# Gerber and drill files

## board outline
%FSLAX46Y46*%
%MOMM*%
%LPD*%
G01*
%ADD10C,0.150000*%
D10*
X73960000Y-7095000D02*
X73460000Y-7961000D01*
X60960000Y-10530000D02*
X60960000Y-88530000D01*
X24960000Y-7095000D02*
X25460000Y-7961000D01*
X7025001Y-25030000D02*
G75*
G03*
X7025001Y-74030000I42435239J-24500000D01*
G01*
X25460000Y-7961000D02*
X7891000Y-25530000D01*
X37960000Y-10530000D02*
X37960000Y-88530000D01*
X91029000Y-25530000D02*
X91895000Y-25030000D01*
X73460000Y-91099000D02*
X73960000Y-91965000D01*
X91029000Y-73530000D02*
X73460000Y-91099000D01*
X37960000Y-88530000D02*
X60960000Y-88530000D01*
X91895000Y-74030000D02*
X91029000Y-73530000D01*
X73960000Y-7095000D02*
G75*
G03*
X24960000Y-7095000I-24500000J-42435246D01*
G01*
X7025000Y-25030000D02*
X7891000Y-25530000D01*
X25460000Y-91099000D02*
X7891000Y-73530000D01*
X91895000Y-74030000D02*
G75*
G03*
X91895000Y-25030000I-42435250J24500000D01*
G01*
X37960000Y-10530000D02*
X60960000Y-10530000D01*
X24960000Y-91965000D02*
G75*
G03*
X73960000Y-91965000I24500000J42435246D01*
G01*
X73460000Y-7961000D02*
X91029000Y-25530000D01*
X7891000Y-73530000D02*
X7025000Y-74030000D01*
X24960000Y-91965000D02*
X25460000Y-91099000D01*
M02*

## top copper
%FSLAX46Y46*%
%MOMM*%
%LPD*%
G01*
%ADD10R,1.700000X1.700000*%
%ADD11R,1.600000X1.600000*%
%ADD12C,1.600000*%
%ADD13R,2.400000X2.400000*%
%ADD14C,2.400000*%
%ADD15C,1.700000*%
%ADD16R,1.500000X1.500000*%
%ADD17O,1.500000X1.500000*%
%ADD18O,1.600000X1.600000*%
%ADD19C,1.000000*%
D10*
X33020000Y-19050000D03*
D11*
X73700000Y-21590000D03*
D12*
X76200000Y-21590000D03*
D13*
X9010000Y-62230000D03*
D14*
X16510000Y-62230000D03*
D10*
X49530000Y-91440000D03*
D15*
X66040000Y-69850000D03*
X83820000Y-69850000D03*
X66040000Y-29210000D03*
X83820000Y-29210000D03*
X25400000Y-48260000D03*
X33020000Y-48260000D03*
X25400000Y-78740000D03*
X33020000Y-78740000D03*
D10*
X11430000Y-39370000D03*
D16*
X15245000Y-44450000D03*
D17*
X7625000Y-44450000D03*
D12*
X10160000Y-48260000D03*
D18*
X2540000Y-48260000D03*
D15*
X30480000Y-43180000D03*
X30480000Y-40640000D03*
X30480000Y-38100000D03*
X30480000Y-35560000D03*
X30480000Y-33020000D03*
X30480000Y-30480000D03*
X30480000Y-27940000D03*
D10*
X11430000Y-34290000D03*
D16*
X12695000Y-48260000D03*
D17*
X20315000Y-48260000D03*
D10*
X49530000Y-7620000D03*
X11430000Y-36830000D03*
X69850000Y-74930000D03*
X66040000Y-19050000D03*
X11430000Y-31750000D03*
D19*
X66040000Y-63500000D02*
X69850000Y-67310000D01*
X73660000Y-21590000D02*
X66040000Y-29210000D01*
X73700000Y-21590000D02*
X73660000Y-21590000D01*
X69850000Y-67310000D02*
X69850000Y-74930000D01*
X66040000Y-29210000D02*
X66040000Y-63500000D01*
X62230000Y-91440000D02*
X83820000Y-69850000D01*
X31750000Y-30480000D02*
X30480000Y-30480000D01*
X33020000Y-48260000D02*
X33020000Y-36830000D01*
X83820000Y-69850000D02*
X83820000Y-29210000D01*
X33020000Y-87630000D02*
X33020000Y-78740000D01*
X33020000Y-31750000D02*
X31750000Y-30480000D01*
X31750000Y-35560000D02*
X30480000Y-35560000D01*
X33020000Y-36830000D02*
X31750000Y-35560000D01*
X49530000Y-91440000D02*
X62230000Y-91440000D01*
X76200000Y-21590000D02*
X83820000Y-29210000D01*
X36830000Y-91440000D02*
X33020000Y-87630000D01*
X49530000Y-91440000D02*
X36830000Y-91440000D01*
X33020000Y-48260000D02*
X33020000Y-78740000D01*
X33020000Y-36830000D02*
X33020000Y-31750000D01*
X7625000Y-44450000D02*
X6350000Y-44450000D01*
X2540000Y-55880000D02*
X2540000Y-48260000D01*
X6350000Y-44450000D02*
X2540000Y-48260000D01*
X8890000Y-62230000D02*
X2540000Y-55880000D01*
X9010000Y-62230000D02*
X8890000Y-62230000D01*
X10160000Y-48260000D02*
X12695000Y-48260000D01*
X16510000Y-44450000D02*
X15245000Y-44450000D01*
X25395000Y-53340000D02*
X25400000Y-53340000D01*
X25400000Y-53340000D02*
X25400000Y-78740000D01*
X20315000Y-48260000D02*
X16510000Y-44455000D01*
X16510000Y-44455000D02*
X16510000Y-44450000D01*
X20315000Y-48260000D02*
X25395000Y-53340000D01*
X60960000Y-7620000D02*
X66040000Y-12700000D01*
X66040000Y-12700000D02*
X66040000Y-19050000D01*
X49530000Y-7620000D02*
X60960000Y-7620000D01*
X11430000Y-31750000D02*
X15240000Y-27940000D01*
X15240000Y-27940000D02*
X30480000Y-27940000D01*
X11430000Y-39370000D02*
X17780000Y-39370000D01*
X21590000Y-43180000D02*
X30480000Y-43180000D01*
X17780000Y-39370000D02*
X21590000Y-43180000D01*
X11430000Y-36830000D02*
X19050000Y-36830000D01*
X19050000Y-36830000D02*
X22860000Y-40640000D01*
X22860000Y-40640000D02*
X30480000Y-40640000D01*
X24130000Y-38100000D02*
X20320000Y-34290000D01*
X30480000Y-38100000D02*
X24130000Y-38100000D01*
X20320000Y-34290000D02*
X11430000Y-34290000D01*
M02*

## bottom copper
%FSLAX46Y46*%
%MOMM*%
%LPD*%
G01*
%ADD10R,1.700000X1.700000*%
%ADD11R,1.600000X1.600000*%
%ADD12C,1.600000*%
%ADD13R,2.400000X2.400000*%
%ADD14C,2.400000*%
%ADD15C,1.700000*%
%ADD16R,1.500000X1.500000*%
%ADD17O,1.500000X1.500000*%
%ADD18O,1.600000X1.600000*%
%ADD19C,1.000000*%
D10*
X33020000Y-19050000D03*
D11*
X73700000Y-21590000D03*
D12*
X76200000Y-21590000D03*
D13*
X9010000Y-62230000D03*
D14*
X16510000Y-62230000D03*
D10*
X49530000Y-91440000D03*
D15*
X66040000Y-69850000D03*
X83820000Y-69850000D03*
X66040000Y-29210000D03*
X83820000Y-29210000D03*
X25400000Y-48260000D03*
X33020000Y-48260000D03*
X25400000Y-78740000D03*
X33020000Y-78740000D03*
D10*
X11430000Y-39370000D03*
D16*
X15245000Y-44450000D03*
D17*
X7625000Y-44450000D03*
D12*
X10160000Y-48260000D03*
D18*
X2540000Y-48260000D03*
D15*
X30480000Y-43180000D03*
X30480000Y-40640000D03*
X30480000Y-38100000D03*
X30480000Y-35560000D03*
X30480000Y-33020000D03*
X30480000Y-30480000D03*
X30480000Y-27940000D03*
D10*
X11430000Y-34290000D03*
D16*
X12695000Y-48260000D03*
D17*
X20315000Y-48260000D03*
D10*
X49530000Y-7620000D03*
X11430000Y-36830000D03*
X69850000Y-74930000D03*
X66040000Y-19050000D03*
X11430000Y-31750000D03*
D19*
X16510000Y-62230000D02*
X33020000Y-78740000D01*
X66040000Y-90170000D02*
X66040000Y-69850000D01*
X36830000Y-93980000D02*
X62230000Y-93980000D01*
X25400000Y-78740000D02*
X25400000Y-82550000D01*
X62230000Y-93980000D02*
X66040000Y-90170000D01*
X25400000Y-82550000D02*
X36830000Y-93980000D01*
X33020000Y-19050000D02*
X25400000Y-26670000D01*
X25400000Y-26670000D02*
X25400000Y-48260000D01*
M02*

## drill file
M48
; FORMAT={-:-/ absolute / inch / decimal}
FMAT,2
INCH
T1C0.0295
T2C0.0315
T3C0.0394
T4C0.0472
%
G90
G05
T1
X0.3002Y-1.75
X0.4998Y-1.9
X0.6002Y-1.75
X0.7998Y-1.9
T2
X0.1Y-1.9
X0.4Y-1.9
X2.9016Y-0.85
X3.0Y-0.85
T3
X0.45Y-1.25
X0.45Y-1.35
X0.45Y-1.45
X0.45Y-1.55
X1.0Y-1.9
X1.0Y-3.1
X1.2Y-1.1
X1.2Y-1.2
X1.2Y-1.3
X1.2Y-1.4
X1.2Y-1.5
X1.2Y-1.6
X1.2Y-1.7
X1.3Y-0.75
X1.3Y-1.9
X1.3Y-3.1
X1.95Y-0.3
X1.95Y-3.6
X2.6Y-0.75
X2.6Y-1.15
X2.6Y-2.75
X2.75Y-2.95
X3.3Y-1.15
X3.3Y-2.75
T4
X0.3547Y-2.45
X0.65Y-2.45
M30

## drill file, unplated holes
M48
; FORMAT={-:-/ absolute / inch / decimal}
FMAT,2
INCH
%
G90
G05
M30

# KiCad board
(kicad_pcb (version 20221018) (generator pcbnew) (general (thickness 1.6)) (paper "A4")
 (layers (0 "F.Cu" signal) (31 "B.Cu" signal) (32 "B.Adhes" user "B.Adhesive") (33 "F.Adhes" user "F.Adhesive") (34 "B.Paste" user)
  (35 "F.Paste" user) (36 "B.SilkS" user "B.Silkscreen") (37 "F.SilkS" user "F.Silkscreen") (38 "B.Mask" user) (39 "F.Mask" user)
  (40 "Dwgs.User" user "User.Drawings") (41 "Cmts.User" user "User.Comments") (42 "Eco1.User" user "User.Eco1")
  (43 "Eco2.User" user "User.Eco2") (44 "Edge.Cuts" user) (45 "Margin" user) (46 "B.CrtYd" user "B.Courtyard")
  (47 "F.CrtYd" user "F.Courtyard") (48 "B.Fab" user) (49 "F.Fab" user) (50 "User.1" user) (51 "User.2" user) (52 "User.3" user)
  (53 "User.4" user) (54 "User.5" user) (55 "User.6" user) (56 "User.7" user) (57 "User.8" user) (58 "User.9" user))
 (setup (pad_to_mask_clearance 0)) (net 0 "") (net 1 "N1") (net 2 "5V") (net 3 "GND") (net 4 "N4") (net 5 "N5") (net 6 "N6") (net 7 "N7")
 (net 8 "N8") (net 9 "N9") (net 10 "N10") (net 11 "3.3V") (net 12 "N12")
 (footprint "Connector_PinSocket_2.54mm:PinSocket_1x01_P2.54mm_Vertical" (layer "F.Cu") (at 33.02 19.05)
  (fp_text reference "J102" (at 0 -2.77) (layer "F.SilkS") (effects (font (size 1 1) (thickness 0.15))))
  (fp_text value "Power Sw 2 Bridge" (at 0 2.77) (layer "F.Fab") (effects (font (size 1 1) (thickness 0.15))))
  (pad "1" thru_hole rect (at 0 0) (size 1.7 1.7) (drill 1) (layers "*.Cu" "*.Mask") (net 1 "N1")))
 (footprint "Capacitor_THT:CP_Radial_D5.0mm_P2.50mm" (layer "F.Cu") (at 73.7 21.59)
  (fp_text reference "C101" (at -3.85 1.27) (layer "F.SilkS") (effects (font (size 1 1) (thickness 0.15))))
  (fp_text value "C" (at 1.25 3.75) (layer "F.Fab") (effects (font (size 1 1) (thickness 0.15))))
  (pad "1" thru_hole rect (at 0 0) (size 1.6 1.6) (drill 0.8) (layers "*.Cu" "*.Mask") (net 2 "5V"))
  (pad "2" thru_hole circle (at 2.5 0) (size 1.6 1.6) (drill 0.8) (layers "*.Cu" "*.Mask") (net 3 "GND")))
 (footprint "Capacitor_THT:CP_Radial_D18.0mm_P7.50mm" (layer "F.Cu") (at 9.01 62.23)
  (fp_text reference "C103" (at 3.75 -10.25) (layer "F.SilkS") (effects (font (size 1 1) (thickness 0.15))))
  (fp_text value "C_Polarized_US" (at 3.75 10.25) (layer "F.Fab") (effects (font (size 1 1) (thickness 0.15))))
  (pad "1" thru_hole rect (at 0 0) (size 2.4 2.4) (drill 1.2) (layers "*.Cu" "*.Mask") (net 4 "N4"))
  (pad "2" thru_hole circle (at 7.5 0) (size 2.4 2.4) (drill 1.2) (layers "*.Cu" "*.Mask") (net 3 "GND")))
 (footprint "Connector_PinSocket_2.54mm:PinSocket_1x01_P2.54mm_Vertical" (layer "F.Cu") (at 49.53 91.44)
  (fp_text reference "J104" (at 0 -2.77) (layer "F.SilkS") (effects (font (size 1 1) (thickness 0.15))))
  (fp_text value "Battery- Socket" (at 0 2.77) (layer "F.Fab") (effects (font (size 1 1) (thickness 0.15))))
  (pad "1" thru_hole rect (at 0 0) (size 1.7 1.7) (drill 1) (layers "*.Cu" "*.Mask") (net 3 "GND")))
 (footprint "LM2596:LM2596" (layer "F.Cu") (at 76.2 49.53 90)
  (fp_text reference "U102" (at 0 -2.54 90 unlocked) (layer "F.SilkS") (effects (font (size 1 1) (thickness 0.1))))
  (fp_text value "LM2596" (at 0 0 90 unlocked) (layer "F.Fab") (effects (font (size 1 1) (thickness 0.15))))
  (pad "1" thru_hole circle (at -20.32 -10.16 90) (size 1.7 1.7) (drill 1) (layers "*.Cu" "*.Mask") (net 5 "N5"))
  (pad "2" thru_hole circle (at -20.32 7.62 90) (size 1.7 1.7) (drill 1) (layers "*.Cu" "*.Mask") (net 3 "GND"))
  (pad "3" thru_hole circle (at 20.32 -10.16 90) (size 1.7 1.7) (drill 1) (layers "*.Cu" "*.Mask") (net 2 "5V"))
  (pad "4" thru_hole circle (at 20.32 7.62 90) (size 1.7 1.7) (drill 1) (layers "*.Cu" "*.Mask") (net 3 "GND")))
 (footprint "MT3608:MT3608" (layer "F.Cu") (at 27.94 63.5 90)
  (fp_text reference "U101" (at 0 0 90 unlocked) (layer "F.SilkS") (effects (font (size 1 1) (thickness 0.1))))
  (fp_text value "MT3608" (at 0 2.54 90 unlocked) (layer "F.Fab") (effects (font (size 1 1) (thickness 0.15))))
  (pad "1" thru_hole circle (at 15.24 -2.54 90) (size 1.7 1.7) (drill 1) (layers "*.Cu" "*.Mask") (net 1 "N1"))
  (pad "2" thru_hole circle (at 15.24 5.08 90) (size 1.7 1.7) (drill 1) (layers "*.Cu" "*.Mask") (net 3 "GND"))
  (pad "3" thru_hole circle (at -15.24 -2.54 90) (size 1.7 1.7) (drill 1) (layers "*.Cu" "*.Mask") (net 5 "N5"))
  (pad "4" thru_hole circle (at -15.24 5.08 90) (size 1.7 1.7) (drill 1) (layers "*.Cu" "*.Mask") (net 3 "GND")))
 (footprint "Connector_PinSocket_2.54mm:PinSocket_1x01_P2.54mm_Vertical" (layer "F.Cu") (at 11.43 39.37)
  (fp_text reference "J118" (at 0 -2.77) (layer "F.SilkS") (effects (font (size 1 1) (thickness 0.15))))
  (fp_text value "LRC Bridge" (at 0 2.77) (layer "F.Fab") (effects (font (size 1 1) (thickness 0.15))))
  (pad "1" thru_hole rect (at 0 0) (size 1.7 1.7) (drill 1) (layers "*.Cu" "*.Mask") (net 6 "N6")))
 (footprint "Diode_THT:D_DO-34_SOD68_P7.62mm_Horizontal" (layer "F.Cu") (at 15.245 44.45 180)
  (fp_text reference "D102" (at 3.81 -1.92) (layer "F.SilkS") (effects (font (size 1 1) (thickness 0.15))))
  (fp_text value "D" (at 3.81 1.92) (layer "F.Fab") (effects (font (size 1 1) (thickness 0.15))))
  (pad "1" thru_hole rect (at 0 0 180) (size 1.5 1.5) (drill 0.75) (layers "*.Cu" "*.Mask") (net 5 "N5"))
  (pad "2" thru_hole oval (at 7.62 0 180) (size 1.5 1.5) (drill 0.75) (layers "*.Cu" "*.Mask") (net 4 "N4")))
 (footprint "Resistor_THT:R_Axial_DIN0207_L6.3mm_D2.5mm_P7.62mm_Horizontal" (layer "F.Cu") (at 10.16 48.26 180)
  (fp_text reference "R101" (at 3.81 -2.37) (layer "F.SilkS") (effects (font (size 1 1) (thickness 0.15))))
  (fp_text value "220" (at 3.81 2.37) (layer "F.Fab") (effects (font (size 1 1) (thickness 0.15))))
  (pad "1" thru_hole circle (at 0 0 180) (size 1.6 1.6) (drill 0.8) (layers "*.Cu" "*.Mask") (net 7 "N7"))
  (pad "2" thru_hole oval (at 7.62 0 180) (size 1.6 1.6) (drill 0.8) (layers "*.Cu" "*.Mask") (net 4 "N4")))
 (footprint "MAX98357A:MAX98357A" (layer "F.Cu") (at 24.13 35.56 90)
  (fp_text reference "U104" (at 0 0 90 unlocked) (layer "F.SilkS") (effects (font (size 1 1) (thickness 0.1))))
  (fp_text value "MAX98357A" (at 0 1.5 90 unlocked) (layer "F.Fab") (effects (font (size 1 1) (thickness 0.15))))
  (pad "1" thru_hole circle (at -7.62 6.35 90) (size 1.7 1.7) (drill 1) (layers "*.Cu" "*.Mask") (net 6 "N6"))
  (pad "2" thru_hole circle (at -5.08 6.35 90) (size 1.7 1.7) (drill 1) (layers "*.Cu" "*.Mask") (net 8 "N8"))
  (pad "3" thru_hole circle (at -2.54 6.35 90) (size 1.7 1.7) (drill 1) (layers "*.Cu" "*.Mask") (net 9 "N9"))
  (pad "4" thru_hole circle (at 0 6.35 90) (size 1.7 1.7) (drill 1) (layers "*.Cu" "*.Mask") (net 3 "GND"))
  (pad "5" thru_hole circle (at 2.54 6.35 90) (size 1.7 1.7) (drill 1) (layers "*.Cu" "*.Mask") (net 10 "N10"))
  (pad "6" thru_hole circle (at 5.08 6.35 90) (size 1.7 1.7) (drill 1) (layers "*.Cu" "*.Mask") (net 3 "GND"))
  (pad "7" thru_hole circle (at 7.62 6.35 90) (size 1.7 1.7) (drill 1) (layers "*.Cu" "*.Mask") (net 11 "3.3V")))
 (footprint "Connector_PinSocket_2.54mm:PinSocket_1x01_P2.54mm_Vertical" (layer "F.Cu") (at 11.43 34.29)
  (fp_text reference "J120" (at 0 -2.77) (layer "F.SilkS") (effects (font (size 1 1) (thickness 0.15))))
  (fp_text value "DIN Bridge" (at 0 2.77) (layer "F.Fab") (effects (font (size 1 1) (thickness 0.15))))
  (pad "1" thru_hole rect (at 0 0) (size 1.7 1.7) (drill 1) (layers "*.Cu" "*.Mask") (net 9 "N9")))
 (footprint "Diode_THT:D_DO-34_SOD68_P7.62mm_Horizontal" (layer "F.Cu") (at 12.695 48.26)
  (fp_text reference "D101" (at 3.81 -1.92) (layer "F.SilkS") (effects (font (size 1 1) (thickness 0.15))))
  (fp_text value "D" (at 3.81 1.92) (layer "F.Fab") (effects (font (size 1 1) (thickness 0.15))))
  (pad "1" thru_hole rect (at 0 0) (size 1.5 1.5) (drill 0.75) (layers "*.Cu" "*.Mask") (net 7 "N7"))
  (pad "2" thru_hole oval (at 7.62 0) (size 1.5 1.5) (drill 0.75) (layers "*.Cu" "*.Mask") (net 5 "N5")))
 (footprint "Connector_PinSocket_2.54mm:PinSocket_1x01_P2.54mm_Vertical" (layer "F.Cu") (at 49.53 7.62)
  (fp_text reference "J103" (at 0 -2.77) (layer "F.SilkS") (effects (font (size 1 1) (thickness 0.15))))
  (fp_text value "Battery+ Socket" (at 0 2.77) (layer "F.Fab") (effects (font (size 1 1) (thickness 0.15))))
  (pad "1" thru_hole rect (at 0 0) (size 1.7 1.7) (drill 1) (layers "*.Cu" "*.Mask") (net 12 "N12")))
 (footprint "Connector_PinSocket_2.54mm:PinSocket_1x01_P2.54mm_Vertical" (layer "F.Cu") (at 11.43 36.83)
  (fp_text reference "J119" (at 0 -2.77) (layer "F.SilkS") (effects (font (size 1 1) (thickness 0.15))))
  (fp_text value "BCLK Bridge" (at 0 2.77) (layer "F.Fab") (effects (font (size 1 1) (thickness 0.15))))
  (pad "1" thru_hole rect (at 0 0) (size 1.7 1.7) (drill 1) (layers "*.Cu" "*.Mask") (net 8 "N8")))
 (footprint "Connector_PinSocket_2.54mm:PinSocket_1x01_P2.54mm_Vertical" (layer "F.Cu") (at 69.85 74.93)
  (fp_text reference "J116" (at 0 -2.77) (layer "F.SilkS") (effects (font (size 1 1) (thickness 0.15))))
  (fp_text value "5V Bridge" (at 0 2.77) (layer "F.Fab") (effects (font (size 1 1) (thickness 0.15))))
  (pad "1" thru_hole rect (at 0 0) (size 1.7 1.7) (drill 1) (layers "*.Cu" "*.Mask") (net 2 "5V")))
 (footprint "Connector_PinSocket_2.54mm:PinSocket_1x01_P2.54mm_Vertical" (layer "F.Cu") (at 66.04 19.05)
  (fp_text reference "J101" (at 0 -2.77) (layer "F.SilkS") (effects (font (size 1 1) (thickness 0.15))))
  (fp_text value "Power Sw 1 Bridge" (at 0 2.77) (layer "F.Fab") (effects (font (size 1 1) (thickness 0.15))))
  (pad "1" thru_hole rect (at 0 0) (size 1.7 1.7) (drill 1) (layers "*.Cu" "*.Mask") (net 12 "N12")))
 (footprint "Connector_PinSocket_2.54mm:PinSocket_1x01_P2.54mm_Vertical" (layer "F.Cu") (at 11.43 31.75)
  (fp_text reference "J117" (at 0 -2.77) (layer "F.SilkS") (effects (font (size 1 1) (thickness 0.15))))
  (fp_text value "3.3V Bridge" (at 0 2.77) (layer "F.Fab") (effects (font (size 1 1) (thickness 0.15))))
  (pad "1" thru_hole rect (at 0 0) (size 1.7 1.7) (drill 1) (layers "*.Cu" "*.Mask") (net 11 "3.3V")))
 (gr_line (start 73.96 7.095) (end 73.46 7.961) (stroke (width 0.15) (type default)) (layer "Edge.Cuts"))
 (gr_line (start 60.96 10.53) (end 60.96 88.53) (stroke (width 0.15) (type default)) (layer "Edge.Cuts"))
 (gr_line (start 24.96 7.095) (end 25.46 7.961) (stroke (width 0.15) (type default)) (layer "Edge.Cuts"))
 (gr_arc (start 7.025 74.03) (mid 0.460244 49.53) (end 7.025 25.03) (stroke (width 0.15) (type default)) (layer "Edge.Cuts"))
 (gr_line (start 25.46 7.961) (end 7.891 25.53) (stroke (width 0.15) (type default)) (layer "Edge.Cuts"))
 (gr_line (start 37.96 10.53) (end 37.96 88.53) (stroke (width 0.15) (type default)) (layer "Edge.Cuts"))
 (gr_line (start 91.029 25.53) (end 91.895 25.03) (stroke (width 0.15) (type default)) (layer "Edge.Cuts"))
 (gr_line (start 73.46 91.099) (end 73.96 91.965) (stroke (width 0.15) (type default)) (layer "Edge.Cuts"))
 (gr_line (start 91.029 73.53) (end 73.46 91.099) (stroke (width 0.15) (type default)) (layer "Edge.Cuts"))
 (gr_line (start 37.96 88.53) (end 60.96 88.53) (stroke (width 0.15) (type default)) (layer "Edge.Cuts"))
 (gr_line (start 91.895 74.03) (end 91.029 73.53) (stroke (width 0.15) (type default)) (layer "Edge.Cuts"))
 (gr_arc (start 24.96 7.095) (mid 49.46 0.530245) (end 73.96 7.095) (stroke (width 0.15) (type default)) (layer "Edge.Cuts"))
 (gr_line (start 7.025 25.03) (end 7.891 25.53) (stroke (width 0.15) (type default)) (layer "Edge.Cuts"))
 (gr_line (start 25.46 91.099) (end 7.891 73.53) (stroke (width 0.15) (type default)) (layer "Edge.Cuts"))
 (gr_arc (start 91.895 25.03) (mid 98.459755 49.53) (end 91.895 74.03) (stroke (width 0.15) (type default)) (layer "Edge.Cuts"))
 (gr_line (start 37.96 10.53) (end 60.96 10.53) (stroke (width 0.15) (type default)) (layer "Edge.Cuts"))
 (gr_arc (start 73.96 91.965) (mid 49.46 98.529755) (end 24.96 91.965) (stroke (width 0.15) (type default)) (layer "Edge.Cuts"))
 (gr_line (start 73.46 7.961) (end 91.029 25.53) (stroke (width 0.15) (type default)) (layer "Edge.Cuts"))
 (gr_line (start 7.891 73.53) (end 7.025 74.03) (stroke (width 0.15) (type default)) (layer "Edge.Cuts"))
 (gr_line (start 24.96 91.965) (end 25.46 91.099) (stroke (width 0.15) (type default)) (layer "Edge.Cuts"))
 (segment (start 66.04 63.5) (end 69.85 67.31) (width 1) (layer "F.Cu") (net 2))
 (segment (start 73.66 21.59) (end 66.04 29.21) (width 1) (layer "F.Cu") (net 2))
 (segment (start 73.7 21.59) (end 73.66 21.59) (width 1) (layer "F.Cu") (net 2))
 (segment (start 69.85 67.31) (end 69.85 74.93) (width 1) (layer "F.Cu") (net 2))
 (segment (start 66.04 29.21) (end 66.04 63.5) (width 1) (layer "F.Cu") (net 2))
 (segment (start 62.23 91.44) (end 83.82 69.85) (width 1) (layer "F.Cu") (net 3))
 (segment (start 31.75 30.48) (end 30.48 30.48) (width 1) (layer "F.Cu") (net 3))
 (segment (start 33.02 48.26) (end 33.02 36.83) (width 1) (layer "F.Cu") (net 3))
 (segment (start 83.82 69.85) (end 83.82 29.21) (width 1) (layer "F.Cu") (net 3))
 (segment (start 33.02 87.63) (end 33.02 78.74) (width 1) (layer "F.Cu") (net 3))
 (segment (start 33.02 31.75) (end 31.75 30.48) (width 1) (layer "F.Cu") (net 3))
 (segment (start 31.75 35.56) (end 30.48 35.56) (width 1) (layer "F.Cu") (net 3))
 (segment (start 33.02 36.83) (end 31.75 35.56) (width 1) (layer "F.Cu") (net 3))
 (segment (start 49.53 91.44) (end 62.23 91.44) (width 1) (layer "F.Cu") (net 3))
 (segment (start 76.2 21.59) (end 83.82 29.21) (width 1) (layer "F.Cu") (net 3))
 (segment (start 36.83 91.44) (end 33.02 87.63) (width 1) (layer "F.Cu") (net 3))
 (segment (start 49.53 91.44) (end 36.83 91.44) (width 1) (layer "F.Cu") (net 3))
 (segment (start 33.02 48.26) (end 33.02 78.74) (width 1) (layer "F.Cu") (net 3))
 (segment (start 33.02 36.83) (end 33.02 31.75) (width 1) (layer "F.Cu") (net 3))
 (segment (start 16.51 62.23) (end 33.02 78.74) (width 1) (layer "B.Cu") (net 3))
 (segment (start 7.625 44.45) (end 6.35 44.45) (width 1) (layer "F.Cu") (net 4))
 (segment (start 2.54 55.88) (end 2.54 48.26) (width 1) (layer "F.Cu") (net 4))
 (segment (start 6.35 44.45) (end 2.54 48.26) (width 1) (layer "F.Cu") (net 4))
 (segment (start 8.89 62.23) (end 2.54 55.88) (width 1) (layer "F.Cu") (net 4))
 (segment (start 9.01 62.23) (end 8.89 62.23) (width 1) (layer "F.Cu") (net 4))
 (segment (start 10.16 48.26) (end 12.695 48.26) (width 1) (layer "F.Cu") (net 7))
 (segment (start 16.51 44.45) (end 15.245 44.45) (width 1) (layer "F.Cu") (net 5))
 (segment (start 25.395 53.34) (end 25.4 53.34) (width 1) (layer "F.Cu") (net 5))
 (segment (start 25.4 53.34) (end 25.4 78.74) (width 1) (layer "F.Cu") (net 5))
 (segment (start 20.315 48.26) (end 16.51 44.455) (width 1) (layer "F.Cu") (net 5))
 (segment (start 16.51 44.455) (end 16.51 44.45) (width 1) (layer "F.Cu") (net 5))
 (segment (start 20.315 48.26) (end 25.395 53.34) (width 1) (layer "F.Cu") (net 5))
 (segment (start 66.04 90.17) (end 66.04 69.85) (width 1) (layer "B.Cu") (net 5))
 (segment (start 36.83 93.98) (end 62.23 93.98) (width 1) (layer "B.Cu") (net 5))
 (segment (start 25.4 78.74) (end 25.4 82.55) (width 1) (layer "B.Cu") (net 5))
 (segment (start 62.23 93.98) (end 66.04 90.17) (width 1) (layer "B.Cu") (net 5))
 (segment (start 25.4 82.55) (end 36.83 93.98) (width 1) (layer "B.Cu") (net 5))
 (segment (start 60.96 7.62) (end 66.04 12.7) (width 1) (layer "F.Cu") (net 12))
 (segment (start 66.04 12.7) (end 66.04 19.05) (width 1) (layer "F.Cu") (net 12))
 (segment (start 49.53 7.62) (end 60.96 7.62) (width 1) (layer "F.Cu") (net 12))
 (segment (start 11.43 31.75) (end 15.24 27.94) (width 1) (layer "F.Cu") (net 11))
 (segment (start 15.24 27.94) (end 30.48 27.94) (width 1) (layer "F.Cu") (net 11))
 (segment (start 11.43 39.37) (end 17.78 39.37) (width 1) (layer "F.Cu") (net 6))
 (segment (start 21.59 43.18) (end 30.48 43.18) (width 1) (layer "F.Cu") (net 6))
 (segment (start 17.78 39.37) (end 21.59 43.18) (width 1) (layer "F.Cu") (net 6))
 (segment (start 11.43 36.83) (end 19.05 36.83) (width 1) (layer "F.Cu") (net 8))
 (segment (start 19.05 36.83) (end 22.86 40.64) (width 1) (layer "F.Cu") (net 8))
 (segment (start 22.86 40.64) (end 30.48 40.64) (width 1) (layer "F.Cu") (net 8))
 (segment (start 24.13 38.1) (end 20.32 34.29) (width 1) (layer "F.Cu") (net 9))
 (segment (start 30.48 38.1) (end 24.13 38.1) (width 1) (layer "F.Cu") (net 9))
 (segment (start 20.32 34.29) (end 11.43 34.29) (width 1) (layer "F.Cu") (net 9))
 (segment (start 33.02 19.05) (end 25.4 26.67) (width 1) (layer "B.Cu") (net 1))
 (segment (start 25.4 26.67) (end 25.4 48.26) (width 1) (layer "B.Cu") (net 1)))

